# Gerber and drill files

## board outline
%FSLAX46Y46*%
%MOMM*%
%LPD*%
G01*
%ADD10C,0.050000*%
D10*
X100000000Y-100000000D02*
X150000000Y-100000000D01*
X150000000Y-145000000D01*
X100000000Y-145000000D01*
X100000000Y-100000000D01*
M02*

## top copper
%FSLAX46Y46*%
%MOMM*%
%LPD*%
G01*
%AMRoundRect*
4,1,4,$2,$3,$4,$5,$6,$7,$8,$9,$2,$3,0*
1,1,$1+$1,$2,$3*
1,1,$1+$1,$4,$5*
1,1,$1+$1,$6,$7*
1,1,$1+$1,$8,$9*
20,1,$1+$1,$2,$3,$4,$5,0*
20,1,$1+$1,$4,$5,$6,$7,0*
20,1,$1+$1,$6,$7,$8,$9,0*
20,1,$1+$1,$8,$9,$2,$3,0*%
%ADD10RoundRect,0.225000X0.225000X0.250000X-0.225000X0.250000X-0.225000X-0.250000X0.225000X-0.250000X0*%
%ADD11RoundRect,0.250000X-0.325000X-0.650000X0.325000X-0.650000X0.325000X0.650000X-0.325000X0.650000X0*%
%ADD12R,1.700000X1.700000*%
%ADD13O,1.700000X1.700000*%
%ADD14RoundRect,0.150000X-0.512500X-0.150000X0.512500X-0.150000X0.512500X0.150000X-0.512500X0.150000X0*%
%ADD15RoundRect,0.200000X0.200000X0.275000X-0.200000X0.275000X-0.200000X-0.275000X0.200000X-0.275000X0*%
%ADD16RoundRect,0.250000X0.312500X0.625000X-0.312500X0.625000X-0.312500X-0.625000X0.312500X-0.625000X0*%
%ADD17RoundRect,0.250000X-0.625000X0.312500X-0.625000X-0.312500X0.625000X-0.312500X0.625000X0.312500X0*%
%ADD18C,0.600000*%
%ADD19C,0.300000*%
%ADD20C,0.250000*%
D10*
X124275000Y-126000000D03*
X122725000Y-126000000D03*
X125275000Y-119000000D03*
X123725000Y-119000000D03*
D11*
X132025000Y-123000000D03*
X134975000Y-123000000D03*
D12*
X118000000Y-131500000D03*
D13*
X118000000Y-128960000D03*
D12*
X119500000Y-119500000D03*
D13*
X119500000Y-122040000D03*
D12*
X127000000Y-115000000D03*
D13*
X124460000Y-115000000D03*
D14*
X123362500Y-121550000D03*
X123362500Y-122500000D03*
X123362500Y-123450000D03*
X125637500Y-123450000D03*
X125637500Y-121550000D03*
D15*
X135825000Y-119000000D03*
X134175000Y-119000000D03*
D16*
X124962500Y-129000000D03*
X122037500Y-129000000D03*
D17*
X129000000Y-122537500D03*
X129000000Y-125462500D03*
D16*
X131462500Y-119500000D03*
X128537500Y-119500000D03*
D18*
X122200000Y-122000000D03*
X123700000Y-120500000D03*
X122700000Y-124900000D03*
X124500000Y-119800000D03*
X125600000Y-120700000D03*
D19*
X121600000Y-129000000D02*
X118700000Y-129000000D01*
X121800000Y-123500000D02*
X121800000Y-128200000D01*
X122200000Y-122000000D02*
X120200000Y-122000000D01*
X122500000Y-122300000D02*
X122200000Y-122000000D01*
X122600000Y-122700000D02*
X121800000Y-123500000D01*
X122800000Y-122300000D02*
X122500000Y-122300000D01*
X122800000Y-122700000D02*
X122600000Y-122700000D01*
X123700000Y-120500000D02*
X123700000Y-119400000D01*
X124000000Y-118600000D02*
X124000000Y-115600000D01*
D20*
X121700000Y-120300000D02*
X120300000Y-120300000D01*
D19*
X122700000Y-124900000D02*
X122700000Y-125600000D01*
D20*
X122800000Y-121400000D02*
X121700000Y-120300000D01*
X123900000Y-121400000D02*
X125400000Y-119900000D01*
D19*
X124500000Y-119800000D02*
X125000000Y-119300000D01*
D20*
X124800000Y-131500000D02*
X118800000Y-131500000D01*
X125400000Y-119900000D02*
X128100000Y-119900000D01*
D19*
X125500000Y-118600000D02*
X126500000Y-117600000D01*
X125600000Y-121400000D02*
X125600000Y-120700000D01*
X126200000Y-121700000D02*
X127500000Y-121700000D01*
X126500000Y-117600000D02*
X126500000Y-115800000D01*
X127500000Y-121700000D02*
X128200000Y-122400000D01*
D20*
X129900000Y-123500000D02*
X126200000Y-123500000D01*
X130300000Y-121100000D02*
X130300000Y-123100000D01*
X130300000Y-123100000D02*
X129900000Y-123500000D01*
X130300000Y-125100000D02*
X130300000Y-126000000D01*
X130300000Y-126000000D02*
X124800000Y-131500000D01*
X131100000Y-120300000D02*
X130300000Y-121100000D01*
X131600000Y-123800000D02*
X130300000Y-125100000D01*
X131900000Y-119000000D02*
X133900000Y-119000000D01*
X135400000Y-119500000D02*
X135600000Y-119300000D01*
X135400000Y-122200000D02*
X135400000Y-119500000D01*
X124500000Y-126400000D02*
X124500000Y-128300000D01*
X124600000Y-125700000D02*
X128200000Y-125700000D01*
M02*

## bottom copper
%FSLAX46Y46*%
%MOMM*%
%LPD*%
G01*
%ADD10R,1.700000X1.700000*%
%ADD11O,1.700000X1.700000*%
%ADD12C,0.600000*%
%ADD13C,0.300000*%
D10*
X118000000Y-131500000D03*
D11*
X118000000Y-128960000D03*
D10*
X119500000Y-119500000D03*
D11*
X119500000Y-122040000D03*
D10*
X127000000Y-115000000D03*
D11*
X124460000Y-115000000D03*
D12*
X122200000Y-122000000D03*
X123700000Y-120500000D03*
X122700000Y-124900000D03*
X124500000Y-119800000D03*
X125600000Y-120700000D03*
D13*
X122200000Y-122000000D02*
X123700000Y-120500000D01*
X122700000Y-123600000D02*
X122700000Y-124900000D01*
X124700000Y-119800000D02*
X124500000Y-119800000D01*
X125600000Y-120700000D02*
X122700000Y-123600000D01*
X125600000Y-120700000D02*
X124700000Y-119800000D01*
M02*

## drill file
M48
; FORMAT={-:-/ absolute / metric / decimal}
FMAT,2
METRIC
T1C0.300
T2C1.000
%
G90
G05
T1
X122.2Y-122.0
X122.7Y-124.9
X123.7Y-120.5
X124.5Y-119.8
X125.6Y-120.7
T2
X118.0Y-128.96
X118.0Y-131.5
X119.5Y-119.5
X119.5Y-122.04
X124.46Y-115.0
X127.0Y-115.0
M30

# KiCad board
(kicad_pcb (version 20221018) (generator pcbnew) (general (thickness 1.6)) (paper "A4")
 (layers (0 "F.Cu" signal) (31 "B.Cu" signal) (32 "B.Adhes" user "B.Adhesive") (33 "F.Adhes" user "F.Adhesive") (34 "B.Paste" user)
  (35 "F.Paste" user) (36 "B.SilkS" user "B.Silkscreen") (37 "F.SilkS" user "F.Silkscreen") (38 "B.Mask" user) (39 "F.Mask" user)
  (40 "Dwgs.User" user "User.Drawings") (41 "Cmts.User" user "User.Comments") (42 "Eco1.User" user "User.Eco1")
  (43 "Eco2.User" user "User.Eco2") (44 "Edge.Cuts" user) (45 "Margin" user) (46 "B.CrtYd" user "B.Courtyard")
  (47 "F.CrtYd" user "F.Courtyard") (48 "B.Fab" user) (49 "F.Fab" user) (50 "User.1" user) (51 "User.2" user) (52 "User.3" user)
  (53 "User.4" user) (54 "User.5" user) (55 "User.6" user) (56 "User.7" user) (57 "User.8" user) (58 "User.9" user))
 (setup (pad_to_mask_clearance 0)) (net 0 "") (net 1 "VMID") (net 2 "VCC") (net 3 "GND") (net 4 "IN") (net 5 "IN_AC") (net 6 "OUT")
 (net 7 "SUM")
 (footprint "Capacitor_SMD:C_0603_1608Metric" (layer "F.Cu") (at 123.5 126 180)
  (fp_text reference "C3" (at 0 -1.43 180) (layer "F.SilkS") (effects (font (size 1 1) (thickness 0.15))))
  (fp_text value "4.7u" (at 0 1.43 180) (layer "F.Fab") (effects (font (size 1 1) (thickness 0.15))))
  (pad "1" smd roundrect (at -0.775 0 180) (size 0.9 0.95) (layers "F.Cu" "F.Paste" "F.Mask") (roundrect_rratio 0.25) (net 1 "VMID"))
  (pad "2" smd roundrect (at 0.775 0 180) (size 0.9 0.95) (layers "F.Cu" "F.Paste" "F.Mask") (roundrect_rratio 0.25) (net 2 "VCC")))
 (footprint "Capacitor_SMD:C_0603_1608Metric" (layer "F.Cu") (at 124.5 119 180)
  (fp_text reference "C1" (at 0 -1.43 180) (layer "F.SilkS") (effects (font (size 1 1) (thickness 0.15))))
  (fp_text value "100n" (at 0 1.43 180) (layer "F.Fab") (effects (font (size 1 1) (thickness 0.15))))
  (pad "1" smd roundrect (at -0.775 0 180) (size 0.9 0.95) (layers "F.Cu" "F.Paste" "F.Mask") (roundrect_rratio 0.25) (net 2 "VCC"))
  (pad "2" smd roundrect (at 0.775 0 180) (size 0.9 0.95) (layers "F.Cu" "F.Paste" "F.Mask") (roundrect_rratio 0.25) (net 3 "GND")))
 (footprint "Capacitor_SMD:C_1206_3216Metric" (layer "F.Cu") (at 133.5 123)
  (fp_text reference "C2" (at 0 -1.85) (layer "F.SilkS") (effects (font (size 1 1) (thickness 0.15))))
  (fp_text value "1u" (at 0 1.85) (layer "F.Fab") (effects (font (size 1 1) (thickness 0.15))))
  (pad "1" smd roundrect (at -1.475 0) (size 1.15 1.8) (layers "F.Cu" "F.Paste" "F.Mask") (roundrect_rratio 0.217391) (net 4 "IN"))
  (pad "2" smd roundrect (at 1.475 0) (size 1.15 1.8) (layers "F.Cu" "F.Paste" "F.Mask") (roundrect_rratio 0.217391) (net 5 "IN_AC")))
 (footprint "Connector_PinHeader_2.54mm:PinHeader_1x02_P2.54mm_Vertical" (layer "F.Cu") (at 118 131.5 180)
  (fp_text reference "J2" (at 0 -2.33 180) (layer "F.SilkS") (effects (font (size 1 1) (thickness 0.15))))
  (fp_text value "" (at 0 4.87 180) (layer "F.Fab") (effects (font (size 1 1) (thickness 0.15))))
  (pad "1" thru_hole rect (at 0 0 180) (size 1.7 1.7) (drill 1) (layers "*.Cu" "*.Mask") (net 4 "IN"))
  (pad "2" thru_hole oval (at 0 2.54 180) (size 1.7 1.7) (drill 1) (layers "*.Cu" "*.Mask") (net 3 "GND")))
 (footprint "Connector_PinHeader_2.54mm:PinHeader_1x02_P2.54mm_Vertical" (layer "F.Cu") (at 119.5 119.5)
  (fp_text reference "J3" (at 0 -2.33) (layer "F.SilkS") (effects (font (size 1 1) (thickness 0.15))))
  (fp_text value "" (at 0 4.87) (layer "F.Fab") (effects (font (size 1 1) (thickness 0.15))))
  (pad "1" thru_hole rect (at 0 0) (size 1.7 1.7) (drill 1) (layers "*.Cu" "*.Mask") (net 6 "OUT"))
  (pad "2" thru_hole oval (at 0 2.54) (size 1.7 1.7) (drill 1) (layers "*.Cu" "*.Mask") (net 3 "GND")))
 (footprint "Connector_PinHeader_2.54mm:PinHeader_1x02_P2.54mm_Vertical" (layer "F.Cu") (at 127 115 -90)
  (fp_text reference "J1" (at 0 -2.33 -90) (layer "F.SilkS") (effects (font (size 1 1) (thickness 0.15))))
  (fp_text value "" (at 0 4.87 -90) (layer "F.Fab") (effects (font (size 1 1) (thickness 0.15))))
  (pad "1" thru_hole rect (at 0 0 270) (size 1.7 1.7) (drill 1) (layers "*.Cu" "*.Mask") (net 2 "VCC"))
  (pad "2" thru_hole oval (at 0 2.54 270) (size 1.7 1.7) (drill 1) (layers "*.Cu" "*.Mask") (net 3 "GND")))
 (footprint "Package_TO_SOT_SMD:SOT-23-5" (layer "F.Cu") (at 124.5 122.5)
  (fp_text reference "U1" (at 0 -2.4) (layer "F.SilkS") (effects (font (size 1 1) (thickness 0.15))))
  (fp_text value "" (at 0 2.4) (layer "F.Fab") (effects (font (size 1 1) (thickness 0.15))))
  (pad "1" smd roundrect (at -1.1375 -0.95) (size 1.325 0.6) (layers "F.Cu" "F.Paste" "F.Mask") (roundrect_rratio 0.25) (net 6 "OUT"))
  (pad "2" smd roundrect (at -1.1375 0) (size 1.325 0.6) (layers "F.Cu" "F.Paste" "F.Mask") (roundrect_rratio 0.25) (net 3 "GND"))
  (pad "3" smd roundrect (at -1.1375 0.95) (size 1.325 0.6) (layers "F.Cu" "F.Paste" "F.Mask") (roundrect_rratio 0.25))
  (pad "4" smd roundrect (at 1.1375 0.95) (size 1.325 0.6) (layers "F.Cu" "F.Paste" "F.Mask") (roundrect_rratio 0.25) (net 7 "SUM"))
  (pad "5" smd roundrect (at 1.1375 -0.95) (size 1.325 0.6) (layers "F.Cu" "F.Paste" "F.Mask") (roundrect_rratio 0.25) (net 2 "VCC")))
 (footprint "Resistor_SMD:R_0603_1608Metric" (layer "F.Cu") (at 135 119 180)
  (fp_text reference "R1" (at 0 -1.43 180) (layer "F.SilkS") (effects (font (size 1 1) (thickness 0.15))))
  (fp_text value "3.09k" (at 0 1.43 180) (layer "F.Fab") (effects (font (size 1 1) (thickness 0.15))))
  (pad "1" smd roundrect (at -0.825 0 180) (size 0.8 0.95) (layers "F.Cu" "F.Paste" "F.Mask") (roundrect_rratio 0.25) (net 5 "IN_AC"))
  (pad "2" smd roundrect (at 0.825 0 180) (size 0.8 0.95) (layers "F.Cu" "F.Paste" "F.Mask") (roundrect_rratio 0.25) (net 7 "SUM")))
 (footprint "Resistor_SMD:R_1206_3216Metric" (layer "F.Cu") (at 123.5 129 180)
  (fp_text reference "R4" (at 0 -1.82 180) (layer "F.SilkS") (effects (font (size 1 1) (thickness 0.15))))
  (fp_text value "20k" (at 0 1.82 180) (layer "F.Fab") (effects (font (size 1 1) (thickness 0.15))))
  (pad "1" smd roundrect (at -1.4625 0 180) (size 1.125 1.75) (layers "F.Cu" "F.Paste" "F.Mask") (roundrect_rratio 0.222222) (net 1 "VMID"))
  (pad "2" smd roundrect (at 1.4625 0 180) (size 1.125 1.75) (layers "F.Cu" "F.Paste" "F.Mask") (roundrect_rratio 0.222222) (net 3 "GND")))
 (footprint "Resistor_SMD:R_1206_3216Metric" (layer "F.Cu") (at 129 124 -90)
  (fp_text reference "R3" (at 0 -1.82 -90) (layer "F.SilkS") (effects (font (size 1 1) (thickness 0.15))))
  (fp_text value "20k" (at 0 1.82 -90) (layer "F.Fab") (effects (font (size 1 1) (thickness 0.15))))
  (pad "1" smd roundrect (at -1.4625 0 270) (size 1.125 1.75) (layers "F.Cu" "F.Paste" "F.Mask") (roundrect_rratio 0.222222) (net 2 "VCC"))
  (pad "2" smd roundrect (at 1.4625 0 270) (size 1.125 1.75) (layers "F.Cu" "F.Paste" "F.Mask") (roundrect_rratio 0.222222) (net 1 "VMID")))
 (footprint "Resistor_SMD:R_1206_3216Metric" (layer "F.Cu") (at 130 119.5 180)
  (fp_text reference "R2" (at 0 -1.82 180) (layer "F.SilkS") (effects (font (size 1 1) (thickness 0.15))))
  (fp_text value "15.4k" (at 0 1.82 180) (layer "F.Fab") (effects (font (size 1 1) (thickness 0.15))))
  (pad "1" smd roundrect (at -1.4625 0 180) (size 1.125 1.75) (layers "F.Cu" "F.Paste" "F.Mask") (roundrect_rratio 0.222222) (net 7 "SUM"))
  (pad "2" smd roundrect (at 1.4625 0 180) (size 1.125 1.75) (layers "F.Cu" "F.Paste" "F.Mask") (roundrect_rratio 0.222222) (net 6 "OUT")))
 (gr_rect (start 100 100) (end 150 145) (stroke (width 0.05) (type default)) (fill none) (layer "Edge.Cuts"))
 (segment (start 121.6 129) (end 118.7 129) (width 0.3) (layer "F.Cu") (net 3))
 (segment (start 121.8 123.5) (end 121.8 128.2) (width 0.3) (layer "F.Cu") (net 3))
 (segment (start 122.2 122) (end 120.2 122) (width 0.3) (layer "F.Cu") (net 3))
 (segment (start 122.5 122.3) (end 122.2 122) (width 0.3) (layer "F.Cu") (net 3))
 (segment (start 122.6 122.7) (end 121.8 123.5) (width 0.3) (layer "F.Cu") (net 3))
 (segment (start 122.8 122.3) (end 122.5 122.3) (width 0.3) (layer "F.Cu") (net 3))
 (segment (start 122.8 122.7) (end 122.6 122.7) (width 0.3) (layer "F.Cu") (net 3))
 (segment (start 123.7 120.5) (end 123.7 119.4) (width 0.3) (layer "F.Cu") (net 3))
 (segment (start 124 118.6) (end 124 115.6) (width 0.3) (layer "F.Cu") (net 3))
 (via (at 122.2 122) (size 0.6) (drill 0.3) (layers "F.Cu" "B.Cu") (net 3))
 (via (at 123.7 120.5) (size 0.6) (drill 0.3) (layers "F.Cu" "B.Cu") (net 3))
 (segment (start 121.7 120.3) (end 120.3 120.3) (width 0.25) (layer "F.Cu") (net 6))
 (segment (start 122.2 122) (end 123.7 120.5) (width 0.3) (layer "B.Cu") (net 3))
 (segment (start 122.7 124.9) (end 122.7 125.6) (width 0.3) (layer "F.Cu") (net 2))
 (segment (start 122.8 121.4) (end 121.7 120.3) (width 0.25) (layer "F.Cu") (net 6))
 (segment (start 123.9 121.4) (end 125.4 119.9) (width 0.25) (layer "F.Cu") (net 6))
 (segment (start 124.5 119.8) (end 125 119.3) (width 0.3) (layer "F.Cu") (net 2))
 (segment (start 124.8 131.5) (end 118.8 131.5) (width 0.25) (layer "F.Cu") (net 4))
 (segment (start 125.4 119.9) (end 128.1 119.9) (width 0.25) (layer "F.Cu") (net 6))
 (segment (start 125.5 118.6) (end 126.5 117.6) (width 0.3) (layer "F.Cu") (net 2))
 (segment (start 125.6 121.4) (end 125.6 120.7) (width 0.3) (layer "F.Cu") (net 2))
 (segment (start 126.2 121.7) (end 127.5 121.7) (width 0.3) (layer "F.Cu") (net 2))
 (segment (start 126.5 117.6) (end 126.5 115.8) (width 0.3) (layer "F.Cu") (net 2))
 (segment (start 127.5 121.7) (end 128.2 122.4) (width 0.3) (layer "F.Cu") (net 2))
 (segment (start 129.9 123.5) (end 126.2 123.5) (width 0.25) (layer "F.Cu") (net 7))
 (segment (start 130.3 121.1) (end 130.3 123.1) (width 0.25) (layer "F.Cu") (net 7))
 (segment (start 130.3 123.1) (end 129.9 123.5) (width 0.25) (layer "F.Cu") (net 7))
 (segment (start 130.3 125.1) (end 130.3 126) (width 0.25) (layer "F.Cu") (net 4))
 (segment (start 130.3 126) (end 124.8 131.5) (width 0.25) (layer "F.Cu") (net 4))
 (segment (start 131.1 120.3) (end 130.3 121.1) (width 0.25) (layer "F.Cu") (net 7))
 (segment (start 131.6 123.8) (end 130.3 125.1) (width 0.25) (layer "F.Cu") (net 4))
 (segment (start 131.9 119) (end 133.9 119) (width 0.25) (layer "F.Cu") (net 7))
 (segment (start 135.4 119.5) (end 135.6 119.3) (width 0.25) (layer "F.Cu") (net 5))
 (segment (start 135.4 122.2) (end 135.4 119.5) (width 0.25) (layer "F.Cu") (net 5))
 (via (at 122.7 124.9) (size 0.6) (drill 0.3) (layers "F.Cu" "B.Cu") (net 2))
 (via (at 124.5 119.8) (size 0.6) (drill 0.3) (layers "F.Cu" "B.Cu") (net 2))
 (via (at 125.6 120.7) (size 0.6) (drill 0.3) (layers "F.Cu" "B.Cu") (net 2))
 (segment (start 122.7 123.6) (end 122.7 124.9) (width 0.3) (layer "B.Cu") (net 2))
 (segment (start 124.5 126.4) (end 124.5 128.3) (width 0.25) (layer "F.Cu") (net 1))
 (segment (start 124.6 125.7) (end 128.2 125.7) (width 0.25) (layer "F.Cu") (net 1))
 (segment (start 124.7 119.8) (end 124.5 119.8) (width 0.3) (layer "B.Cu") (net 2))
 (segment (start 125.6 120.7) (end 122.7 123.6) (width 0.3) (layer "B.Cu") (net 2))
 (segment (start 125.6 120.7) (end 124.7 119.8) (width 0.3) (layer "B.Cu") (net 2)))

